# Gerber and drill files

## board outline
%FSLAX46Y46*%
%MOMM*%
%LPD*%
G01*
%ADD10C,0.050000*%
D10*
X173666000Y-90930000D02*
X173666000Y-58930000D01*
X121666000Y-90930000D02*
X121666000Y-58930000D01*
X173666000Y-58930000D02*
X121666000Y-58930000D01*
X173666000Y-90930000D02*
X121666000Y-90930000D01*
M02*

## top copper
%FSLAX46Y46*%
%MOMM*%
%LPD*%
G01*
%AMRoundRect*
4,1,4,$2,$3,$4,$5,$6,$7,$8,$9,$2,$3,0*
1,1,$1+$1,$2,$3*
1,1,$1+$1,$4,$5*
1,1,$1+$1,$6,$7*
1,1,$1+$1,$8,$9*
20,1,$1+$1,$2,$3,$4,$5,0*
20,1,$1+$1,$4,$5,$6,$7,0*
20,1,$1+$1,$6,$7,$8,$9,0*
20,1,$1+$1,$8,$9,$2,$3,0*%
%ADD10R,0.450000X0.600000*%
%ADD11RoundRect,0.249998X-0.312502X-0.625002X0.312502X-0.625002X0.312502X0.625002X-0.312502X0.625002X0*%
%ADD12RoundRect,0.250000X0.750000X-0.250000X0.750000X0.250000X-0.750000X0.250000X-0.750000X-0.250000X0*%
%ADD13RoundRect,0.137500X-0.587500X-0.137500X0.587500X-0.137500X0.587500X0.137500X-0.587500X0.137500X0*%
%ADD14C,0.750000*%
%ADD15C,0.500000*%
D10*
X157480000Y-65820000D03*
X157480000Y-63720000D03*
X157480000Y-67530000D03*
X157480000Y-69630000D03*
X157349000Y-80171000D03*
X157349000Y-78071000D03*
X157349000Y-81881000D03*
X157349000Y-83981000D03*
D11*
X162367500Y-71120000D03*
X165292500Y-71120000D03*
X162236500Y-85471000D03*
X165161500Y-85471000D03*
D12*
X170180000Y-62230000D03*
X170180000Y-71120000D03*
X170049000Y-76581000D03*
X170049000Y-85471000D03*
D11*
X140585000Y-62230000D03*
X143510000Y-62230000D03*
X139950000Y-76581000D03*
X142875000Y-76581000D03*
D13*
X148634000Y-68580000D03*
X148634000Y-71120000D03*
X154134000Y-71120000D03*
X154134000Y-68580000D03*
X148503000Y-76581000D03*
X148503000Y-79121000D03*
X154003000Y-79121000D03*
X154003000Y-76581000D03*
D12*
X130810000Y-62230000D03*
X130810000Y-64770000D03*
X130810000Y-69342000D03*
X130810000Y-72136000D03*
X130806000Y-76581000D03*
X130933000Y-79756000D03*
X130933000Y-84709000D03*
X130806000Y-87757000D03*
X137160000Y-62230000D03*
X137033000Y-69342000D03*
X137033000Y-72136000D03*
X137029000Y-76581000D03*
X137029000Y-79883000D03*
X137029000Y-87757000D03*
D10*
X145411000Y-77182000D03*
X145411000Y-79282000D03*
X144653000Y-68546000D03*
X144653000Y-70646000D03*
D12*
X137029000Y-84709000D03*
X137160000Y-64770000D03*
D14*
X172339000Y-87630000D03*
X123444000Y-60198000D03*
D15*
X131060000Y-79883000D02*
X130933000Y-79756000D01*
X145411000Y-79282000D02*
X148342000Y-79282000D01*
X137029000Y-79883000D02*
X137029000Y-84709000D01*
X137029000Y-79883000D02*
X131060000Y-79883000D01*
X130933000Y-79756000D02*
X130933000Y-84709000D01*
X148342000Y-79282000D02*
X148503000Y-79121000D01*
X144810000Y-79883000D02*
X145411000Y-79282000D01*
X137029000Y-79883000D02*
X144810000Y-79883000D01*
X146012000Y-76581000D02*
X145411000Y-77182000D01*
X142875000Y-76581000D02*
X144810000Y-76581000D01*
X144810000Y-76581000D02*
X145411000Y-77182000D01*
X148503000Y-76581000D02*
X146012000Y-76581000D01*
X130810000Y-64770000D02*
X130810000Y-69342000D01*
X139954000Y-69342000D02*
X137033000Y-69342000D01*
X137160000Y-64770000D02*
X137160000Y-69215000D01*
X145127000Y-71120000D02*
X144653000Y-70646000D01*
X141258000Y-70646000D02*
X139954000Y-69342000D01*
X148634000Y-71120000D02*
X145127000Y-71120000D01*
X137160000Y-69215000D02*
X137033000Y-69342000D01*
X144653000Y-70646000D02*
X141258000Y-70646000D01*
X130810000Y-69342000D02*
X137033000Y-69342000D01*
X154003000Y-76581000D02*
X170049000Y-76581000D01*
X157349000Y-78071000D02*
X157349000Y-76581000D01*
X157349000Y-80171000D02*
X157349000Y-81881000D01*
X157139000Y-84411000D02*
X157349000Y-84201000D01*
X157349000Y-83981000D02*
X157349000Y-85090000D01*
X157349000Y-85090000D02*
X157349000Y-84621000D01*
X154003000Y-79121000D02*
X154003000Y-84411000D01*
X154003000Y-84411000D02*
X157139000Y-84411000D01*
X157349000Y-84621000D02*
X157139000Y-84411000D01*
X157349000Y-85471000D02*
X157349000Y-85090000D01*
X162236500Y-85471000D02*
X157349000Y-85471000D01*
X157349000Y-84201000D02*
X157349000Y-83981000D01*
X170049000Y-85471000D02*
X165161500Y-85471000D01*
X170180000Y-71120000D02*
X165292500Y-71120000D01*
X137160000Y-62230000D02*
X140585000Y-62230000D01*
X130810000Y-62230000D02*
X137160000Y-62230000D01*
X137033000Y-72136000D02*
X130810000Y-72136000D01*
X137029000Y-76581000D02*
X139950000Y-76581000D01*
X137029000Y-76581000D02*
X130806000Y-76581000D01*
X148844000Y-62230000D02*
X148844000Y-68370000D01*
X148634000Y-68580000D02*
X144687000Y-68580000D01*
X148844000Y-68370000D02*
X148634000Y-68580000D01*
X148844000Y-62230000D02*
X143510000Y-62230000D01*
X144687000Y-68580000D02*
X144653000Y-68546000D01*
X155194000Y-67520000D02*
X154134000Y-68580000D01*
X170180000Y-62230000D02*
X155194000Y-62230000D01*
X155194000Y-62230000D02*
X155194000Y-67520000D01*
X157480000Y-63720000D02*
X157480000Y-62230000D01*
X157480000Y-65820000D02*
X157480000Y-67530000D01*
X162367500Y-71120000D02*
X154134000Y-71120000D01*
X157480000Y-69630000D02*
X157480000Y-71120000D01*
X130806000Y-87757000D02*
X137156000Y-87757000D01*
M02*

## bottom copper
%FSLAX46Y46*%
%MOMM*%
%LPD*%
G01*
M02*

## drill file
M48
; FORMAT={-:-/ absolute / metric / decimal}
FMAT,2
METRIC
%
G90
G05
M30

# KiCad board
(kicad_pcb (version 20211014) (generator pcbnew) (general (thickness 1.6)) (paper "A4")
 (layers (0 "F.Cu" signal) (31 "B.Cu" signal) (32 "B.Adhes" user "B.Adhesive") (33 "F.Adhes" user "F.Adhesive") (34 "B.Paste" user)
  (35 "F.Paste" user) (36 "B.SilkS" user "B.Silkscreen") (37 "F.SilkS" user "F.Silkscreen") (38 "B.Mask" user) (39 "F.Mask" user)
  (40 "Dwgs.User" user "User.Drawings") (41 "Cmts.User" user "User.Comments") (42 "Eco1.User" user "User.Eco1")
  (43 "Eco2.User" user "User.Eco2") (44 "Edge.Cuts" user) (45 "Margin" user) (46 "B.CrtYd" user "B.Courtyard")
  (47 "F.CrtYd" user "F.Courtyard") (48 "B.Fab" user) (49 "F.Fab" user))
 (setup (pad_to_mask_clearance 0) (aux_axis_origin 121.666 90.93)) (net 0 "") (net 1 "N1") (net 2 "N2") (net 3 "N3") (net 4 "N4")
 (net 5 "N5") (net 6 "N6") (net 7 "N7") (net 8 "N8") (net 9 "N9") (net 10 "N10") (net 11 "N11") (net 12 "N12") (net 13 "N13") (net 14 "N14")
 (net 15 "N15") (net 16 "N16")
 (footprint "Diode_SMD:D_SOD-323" (layer "F.Cu") (at 157.48 64.77 90)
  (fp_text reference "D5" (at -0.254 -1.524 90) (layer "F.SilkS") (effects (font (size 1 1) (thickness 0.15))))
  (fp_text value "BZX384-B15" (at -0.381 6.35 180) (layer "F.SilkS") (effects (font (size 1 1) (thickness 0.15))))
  (pad "1" smd rect locked (at -1.05 0 90) (size 0.6 0.45) (layers "F.Cu" "F.Paste" "F.Mask") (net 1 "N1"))
  (pad "2" smd rect locked (at 1.05 0 90) (size 0.6 0.45) (layers "F.Cu" "F.Paste" "F.Mask") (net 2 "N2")))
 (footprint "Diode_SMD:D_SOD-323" (layer "F.Cu") (at 157.48 68.58 -90)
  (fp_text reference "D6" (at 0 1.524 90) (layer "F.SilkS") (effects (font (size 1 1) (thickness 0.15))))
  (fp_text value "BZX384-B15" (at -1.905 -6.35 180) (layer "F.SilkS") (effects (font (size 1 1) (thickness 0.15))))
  (pad "1" smd rect locked (at -1.05 0 270) (size 0.6 0.45) (layers "F.Cu" "F.Paste" "F.Mask") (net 1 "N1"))
  (pad "2" smd rect locked (at 1.05 0 270) (size 0.6 0.45) (layers "F.Cu" "F.Paste" "F.Mask") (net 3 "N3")))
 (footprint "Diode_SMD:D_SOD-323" (layer "F.Cu") (at 157.349 79.121 90)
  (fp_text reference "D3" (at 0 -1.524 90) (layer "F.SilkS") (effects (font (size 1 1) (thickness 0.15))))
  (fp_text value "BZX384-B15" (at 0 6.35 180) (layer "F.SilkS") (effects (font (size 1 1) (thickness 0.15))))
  (pad "1" smd rect locked (at -1.05 0 90) (size 0.6 0.45) (layers "F.Cu" "F.Paste" "F.Mask") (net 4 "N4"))
  (pad "2" smd rect locked (at 1.05 0 90) (size 0.6 0.45) (layers "F.Cu" "F.Paste" "F.Mask") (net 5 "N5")))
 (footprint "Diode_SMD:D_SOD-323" (layer "F.Cu") (at 157.349 82.931 -90)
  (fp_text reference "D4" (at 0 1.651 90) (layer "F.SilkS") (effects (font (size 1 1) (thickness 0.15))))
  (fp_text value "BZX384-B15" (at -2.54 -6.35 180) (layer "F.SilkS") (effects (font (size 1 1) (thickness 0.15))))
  (pad "1" smd rect locked (at -1.05 0 270) (size 0.6 0.45) (layers "F.Cu" "F.Paste" "F.Mask") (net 4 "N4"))
  (pad "2" smd rect locked (at 1.05 0 270) (size 0.6 0.45) (layers "F.Cu" "F.Paste" "F.Mask") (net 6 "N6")))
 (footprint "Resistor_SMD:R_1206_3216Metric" (layer "F.Cu") (at 163.83 71.12)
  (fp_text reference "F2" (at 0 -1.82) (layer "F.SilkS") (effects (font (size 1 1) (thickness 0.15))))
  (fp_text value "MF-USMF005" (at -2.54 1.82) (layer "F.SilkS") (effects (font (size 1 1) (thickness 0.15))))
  (pad "1" smd roundrect locked (at -1.4625 0) (size 1.125 1.75) (layers "F.Cu" "F.Paste" "F.Mask") (roundrect_rratio 0.2222204444)
   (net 3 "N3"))
  (pad "2" smd roundrect locked (at 1.4625 0) (size 1.125 1.75) (layers "F.Cu" "F.Paste" "F.Mask") (roundrect_rratio 0.2222204444)
   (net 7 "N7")))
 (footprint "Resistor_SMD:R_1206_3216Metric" (layer "F.Cu") (at 163.699 85.471)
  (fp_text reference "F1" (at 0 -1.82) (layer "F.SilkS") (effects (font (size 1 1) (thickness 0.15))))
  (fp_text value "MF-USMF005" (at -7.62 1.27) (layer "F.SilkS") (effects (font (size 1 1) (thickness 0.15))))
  (pad "1" smd roundrect locked (at -1.4625 0) (size 1.125 1.75) (layers "F.Cu" "F.Paste" "F.Mask") (roundrect_rratio 0.2222204444)
   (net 6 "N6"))
  (pad "2" smd roundrect locked (at 1.4625 0) (size 1.125 1.75) (layers "F.Cu" "F.Paste" "F.Mask") (roundrect_rratio 0.2222204444)
   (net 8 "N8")))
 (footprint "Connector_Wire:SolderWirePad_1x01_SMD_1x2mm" (layer "F.Cu") (at 170.18 62.23 90)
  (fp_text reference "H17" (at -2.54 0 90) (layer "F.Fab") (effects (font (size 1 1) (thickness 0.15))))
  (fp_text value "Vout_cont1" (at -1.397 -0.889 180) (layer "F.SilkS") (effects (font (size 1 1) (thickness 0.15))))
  (pad "1" smd roundrect locked (at 0 0 90) (size 1 2) (layers "F.Cu" "F.Paste" "F.Mask") (roundrect_rratio 0.25) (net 2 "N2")))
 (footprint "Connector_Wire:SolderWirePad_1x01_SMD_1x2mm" (layer "F.Cu") (at 170.18 71.12 90)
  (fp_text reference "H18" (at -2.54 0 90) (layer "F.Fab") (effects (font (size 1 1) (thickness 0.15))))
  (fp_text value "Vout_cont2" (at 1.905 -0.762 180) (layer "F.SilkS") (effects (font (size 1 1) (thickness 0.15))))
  (pad "1" smd roundrect locked (at 0 0 90) (size 1 2) (layers "F.Cu" "F.Paste" "F.Mask") (roundrect_rratio 0.25) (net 7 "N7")))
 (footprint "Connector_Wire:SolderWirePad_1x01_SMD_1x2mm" (layer "F.Cu") (at 170.049 76.581 90)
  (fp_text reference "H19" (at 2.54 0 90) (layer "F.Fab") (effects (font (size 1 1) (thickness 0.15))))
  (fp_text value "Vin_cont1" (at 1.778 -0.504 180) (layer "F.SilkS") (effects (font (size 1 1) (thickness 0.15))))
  (pad "1" smd roundrect locked (at 0 0 90) (size 1 2) (layers "F.Cu" "F.Paste" "F.Mask") (roundrect_rratio 0.25) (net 5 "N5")))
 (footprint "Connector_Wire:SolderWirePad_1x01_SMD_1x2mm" (layer "F.Cu") (at 170.049 85.471 90)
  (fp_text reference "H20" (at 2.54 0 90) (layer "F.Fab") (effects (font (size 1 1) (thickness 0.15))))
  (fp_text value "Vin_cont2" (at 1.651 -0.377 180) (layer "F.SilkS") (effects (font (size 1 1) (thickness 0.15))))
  (pad "1" smd roundrect locked (at 0 0 90) (size 1 2) (layers "F.Cu" "F.Paste" "F.Mask") (roundrect_rratio 0.25) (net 8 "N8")))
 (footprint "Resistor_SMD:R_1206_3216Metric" (layer "F.Cu") (at 142.0475 62.23)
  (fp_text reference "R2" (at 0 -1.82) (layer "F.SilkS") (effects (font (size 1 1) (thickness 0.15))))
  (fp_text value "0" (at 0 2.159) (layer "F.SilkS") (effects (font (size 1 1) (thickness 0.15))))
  (pad "1" smd roundrect locked (at -1.4625 0) (size 1.125 1.75) (layers "F.Cu" "F.Paste" "F.Mask") (roundrect_rratio 0.2222204444)
   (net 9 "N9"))
  (pad "2" smd roundrect locked (at 1.4625 0) (size 1.125 1.75) (layers "F.Cu" "F.Paste" "F.Mask") (roundrect_rratio 0.2222204444)
   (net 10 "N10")))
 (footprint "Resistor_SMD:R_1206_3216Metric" (layer "F.Cu") (at 141.4125 76.581)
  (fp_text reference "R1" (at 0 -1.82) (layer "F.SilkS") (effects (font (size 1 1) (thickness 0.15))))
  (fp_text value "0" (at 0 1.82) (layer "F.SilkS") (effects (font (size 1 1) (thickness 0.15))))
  (pad "1" smd roundrect locked (at -1.4625 0) (size 1.125 1.75) (layers "F.Cu" "F.Paste" "F.Mask") (roundrect_rratio 0.2222204444)
   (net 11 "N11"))
  (pad "2" smd roundrect locked (at 1.4625 0) (size 1.125 1.75) (layers "F.Cu" "F.Paste" "F.Mask") (roundrect_rratio 0.2222204444)
   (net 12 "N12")))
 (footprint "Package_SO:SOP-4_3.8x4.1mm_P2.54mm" (layer "F.Cu") (at 151.384 69.85)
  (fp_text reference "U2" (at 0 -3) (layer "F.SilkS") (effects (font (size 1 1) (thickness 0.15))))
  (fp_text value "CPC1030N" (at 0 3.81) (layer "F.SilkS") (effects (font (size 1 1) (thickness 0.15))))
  (pad "1" smd roundrect locked (at -2.75 -1.27) (size 1.45 0.55) (layers "F.Cu" "F.Paste" "F.Mask") (roundrect_rratio 0.25) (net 10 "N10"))
  (pad "2" smd roundrect locked (at -2.75 1.27) (size 1.45 0.55) (layers "F.Cu" "F.Paste" "F.Mask") (roundrect_rratio 0.25) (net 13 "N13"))
  (pad "3" smd roundrect locked (at 2.75 1.27) (size 1.45 0.55) (layers "F.Cu" "F.Paste" "F.Mask") (roundrect_rratio 0.25) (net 3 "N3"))
  (pad "4" smd roundrect locked (at 2.75 -1.27) (size 1.45 0.55) (layers "F.Cu" "F.Paste" "F.Mask") (roundrect_rratio 0.25) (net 2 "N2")))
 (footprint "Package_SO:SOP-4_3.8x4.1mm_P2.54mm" (layer "F.Cu") (at 151.253 77.851)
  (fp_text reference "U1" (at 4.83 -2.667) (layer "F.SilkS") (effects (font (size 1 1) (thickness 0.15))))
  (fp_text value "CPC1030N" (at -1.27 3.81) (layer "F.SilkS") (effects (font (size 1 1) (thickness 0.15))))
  (pad "1" smd roundrect locked (at -2.75 -1.27) (size 1.45 0.55) (layers "F.Cu" "F.Paste" "F.Mask") (roundrect_rratio 0.25) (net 12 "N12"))
  (pad "2" smd roundrect locked (at -2.75 1.27) (size 1.45 0.55) (layers "F.Cu" "F.Paste" "F.Mask") (roundrect_rratio 0.25) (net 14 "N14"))
  (pad "3" smd roundrect locked (at 2.75 1.27) (size 1.45 0.55) (layers "F.Cu" "F.Paste" "F.Mask") (roundrect_rratio 0.25) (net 6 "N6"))
  (pad "4" smd roundrect locked (at 2.75 -1.27) (size 1.45 0.55) (layers "F.Cu" "F.Paste" "F.Mask") (roundrect_rratio 0.25) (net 5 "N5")))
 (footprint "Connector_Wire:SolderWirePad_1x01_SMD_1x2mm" (layer "F.Cu") (at 130.81 62.23 90)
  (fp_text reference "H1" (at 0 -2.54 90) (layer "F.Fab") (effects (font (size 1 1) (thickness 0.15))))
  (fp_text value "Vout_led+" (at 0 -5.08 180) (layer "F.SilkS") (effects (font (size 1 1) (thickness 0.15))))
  (pad "1" smd roundrect locked (at 0 0 90) (size 1 2) (layers "F.Cu" "F.Paste" "F.Mask") (roundrect_rratio 0.25) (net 9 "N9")))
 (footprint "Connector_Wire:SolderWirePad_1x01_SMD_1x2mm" (layer "F.Cu") (at 130.81 64.77 90)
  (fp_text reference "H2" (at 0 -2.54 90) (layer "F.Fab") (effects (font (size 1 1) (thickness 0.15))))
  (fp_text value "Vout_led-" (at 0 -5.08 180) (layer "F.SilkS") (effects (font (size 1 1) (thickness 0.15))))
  (pad "1" smd roundrect locked (at 0 0 90) (size 1 2) (layers "F.Cu" "F.Paste" "F.Mask") (roundrect_rratio 0.25) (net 13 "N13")))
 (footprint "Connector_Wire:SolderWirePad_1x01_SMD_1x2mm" (layer "F.Cu") (at 130.81 69.342 90)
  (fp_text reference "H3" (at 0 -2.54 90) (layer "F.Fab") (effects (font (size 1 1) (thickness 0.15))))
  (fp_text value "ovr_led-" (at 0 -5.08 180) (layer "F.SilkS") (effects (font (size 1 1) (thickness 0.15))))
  (pad "1" smd roundrect locked (at 0 0 90) (size 1 2) (layers "F.Cu" "F.Paste" "F.Mask") (roundrect_rratio 0.25) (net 13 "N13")))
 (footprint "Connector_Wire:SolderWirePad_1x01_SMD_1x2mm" (layer "F.Cu") (at 130.81 72.136 90)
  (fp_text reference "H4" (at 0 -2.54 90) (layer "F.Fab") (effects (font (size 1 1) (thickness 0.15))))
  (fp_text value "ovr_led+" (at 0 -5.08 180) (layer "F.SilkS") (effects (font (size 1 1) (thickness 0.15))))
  (pad "1" smd roundrect locked (at 0 0 90) (size 1 2) (layers "F.Cu" "F.Paste" "F.Mask") (roundrect_rratio 0.25) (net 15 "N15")))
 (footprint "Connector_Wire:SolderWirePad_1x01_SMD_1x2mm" (layer "F.Cu") (at 130.806 76.581 90)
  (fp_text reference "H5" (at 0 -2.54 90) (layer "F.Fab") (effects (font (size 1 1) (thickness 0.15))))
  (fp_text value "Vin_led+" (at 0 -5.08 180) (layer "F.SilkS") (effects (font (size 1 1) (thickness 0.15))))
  (pad "1" smd roundrect locked (at 0 0 90) (size 1 2) (layers "F.Cu" "F.Paste" "F.Mask") (roundrect_rratio 0.25) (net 11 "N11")))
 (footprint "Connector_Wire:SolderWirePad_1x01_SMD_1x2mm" (layer "F.Cu") (at 130.933 79.756 90)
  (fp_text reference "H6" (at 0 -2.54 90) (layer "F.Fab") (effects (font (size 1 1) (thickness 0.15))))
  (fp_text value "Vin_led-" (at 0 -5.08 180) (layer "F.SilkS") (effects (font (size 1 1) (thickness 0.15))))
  (pad "1" smd roundrect locked (at 0 0 90) (size 1 2) (layers "F.Cu" "F.Paste" "F.Mask") (roundrect_rratio 0.25) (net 14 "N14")))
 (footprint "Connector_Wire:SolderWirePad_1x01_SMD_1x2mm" (layer "F.Cu") (at 130.933 84.709 90)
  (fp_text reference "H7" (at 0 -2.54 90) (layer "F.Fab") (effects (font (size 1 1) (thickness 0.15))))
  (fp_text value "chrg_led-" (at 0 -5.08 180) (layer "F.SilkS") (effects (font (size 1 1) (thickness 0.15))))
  (pad "1" smd roundrect locked (at 0 0 90) (size 1 2) (layers "F.Cu" "F.Paste" "F.Mask") (roundrect_rratio 0.25) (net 14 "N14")))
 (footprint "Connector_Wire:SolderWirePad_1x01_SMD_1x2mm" (layer "F.Cu") (at 130.806 87.757 90)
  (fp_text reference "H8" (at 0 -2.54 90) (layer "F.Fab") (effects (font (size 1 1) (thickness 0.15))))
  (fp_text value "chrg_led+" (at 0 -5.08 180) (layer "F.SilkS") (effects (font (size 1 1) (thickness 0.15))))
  (pad "1" smd roundrect locked (at 0 0 90) (size 1 2) (layers "F.Cu" "F.Paste" "F.Mask") (roundrect_rratio 0.25) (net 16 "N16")))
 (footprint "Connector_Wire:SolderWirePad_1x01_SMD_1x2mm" (layer "F.Cu") (at 137.16 62.23 90)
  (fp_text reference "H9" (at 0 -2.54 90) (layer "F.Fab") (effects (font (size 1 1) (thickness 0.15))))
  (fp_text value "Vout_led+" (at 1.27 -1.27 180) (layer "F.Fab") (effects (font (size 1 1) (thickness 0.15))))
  (pad "1" smd roundrect locked (at 0 0 90) (size 1 2) (layers "F.Cu" "F.Paste" "F.Mask") (roundrect_rratio 0.25) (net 9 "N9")))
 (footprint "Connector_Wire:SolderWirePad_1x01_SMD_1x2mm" (layer "F.Cu") (at 137.033 69.342 90)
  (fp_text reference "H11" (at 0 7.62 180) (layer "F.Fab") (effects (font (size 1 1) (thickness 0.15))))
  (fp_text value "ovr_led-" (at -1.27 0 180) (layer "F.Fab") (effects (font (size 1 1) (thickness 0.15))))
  (pad "1" smd roundrect locked (at 0 0 90) (size 1 2) (layers "F.Cu" "F.Paste" "F.Mask") (roundrect_rratio 0.25) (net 13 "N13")))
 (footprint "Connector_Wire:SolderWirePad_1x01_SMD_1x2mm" (layer "F.Cu") (at 137.033 72.136 90)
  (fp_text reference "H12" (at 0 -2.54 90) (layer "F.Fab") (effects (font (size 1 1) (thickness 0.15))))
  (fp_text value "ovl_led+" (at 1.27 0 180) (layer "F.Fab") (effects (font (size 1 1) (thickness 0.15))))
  (pad "1" smd roundrect locked (at 0 0 90) (size 1 2) (layers "F.Cu" "F.Paste" "F.Mask") (roundrect_rratio 0.25) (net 15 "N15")))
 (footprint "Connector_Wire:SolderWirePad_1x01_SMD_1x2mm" (layer "F.Cu") (at 137.029 76.581 90)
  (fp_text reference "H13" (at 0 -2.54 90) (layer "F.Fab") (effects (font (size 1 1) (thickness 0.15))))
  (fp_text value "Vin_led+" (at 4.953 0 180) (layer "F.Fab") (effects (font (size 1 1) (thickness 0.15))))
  (pad "1" smd roundrect locked (at 0 0 90) (size 1 2) (layers "F.Cu" "F.Paste" "F.Mask") (roundrect_rratio 0.25) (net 11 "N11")))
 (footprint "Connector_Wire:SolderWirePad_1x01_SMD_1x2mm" (layer "F.Cu") (at 137.029 79.883 90)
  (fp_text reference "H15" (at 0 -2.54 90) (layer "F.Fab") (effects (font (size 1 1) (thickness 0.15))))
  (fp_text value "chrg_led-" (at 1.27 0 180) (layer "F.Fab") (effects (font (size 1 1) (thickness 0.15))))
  (pad "1" smd roundrect locked (at 0 0 90) (size 1 2) (layers "F.Cu" "F.Paste" "F.Mask") (roundrect_rratio 0.25) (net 14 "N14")))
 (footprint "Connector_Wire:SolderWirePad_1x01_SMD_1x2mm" (layer "F.Cu") (at 137.029 87.757 90)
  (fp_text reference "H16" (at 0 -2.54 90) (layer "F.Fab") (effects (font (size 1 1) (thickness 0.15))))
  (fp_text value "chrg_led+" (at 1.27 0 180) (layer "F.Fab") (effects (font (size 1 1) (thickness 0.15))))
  (pad "1" smd roundrect locked (at 0 0 90) (size 1 2) (layers "F.Cu" "F.Paste" "F.Mask") (roundrect_rratio 0.25) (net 16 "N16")))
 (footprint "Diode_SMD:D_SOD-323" (layer "F.Cu") (at 145.411 78.232 -90)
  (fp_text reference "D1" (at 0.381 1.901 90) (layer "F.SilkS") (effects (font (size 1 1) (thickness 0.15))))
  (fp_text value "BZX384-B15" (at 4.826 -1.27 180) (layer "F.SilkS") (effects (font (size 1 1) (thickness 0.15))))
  (pad "1" smd rect locked (at -1.05 0 270) (size 0.6 0.45) (layers "F.Cu" "F.Paste" "F.Mask") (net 12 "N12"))
  (pad "2" smd rect locked (at 1.05 0 270) (size 0.6 0.45) (layers "F.Cu" "F.Paste" "F.Mask") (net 14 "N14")))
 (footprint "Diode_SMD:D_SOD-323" (layer "F.Cu") (at 144.653 69.596 -90)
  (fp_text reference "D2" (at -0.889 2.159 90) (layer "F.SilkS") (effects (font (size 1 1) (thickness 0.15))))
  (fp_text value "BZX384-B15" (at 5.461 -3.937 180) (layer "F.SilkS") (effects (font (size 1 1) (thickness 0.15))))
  (pad "1" smd rect locked (at -1.05 0 270) (size 0.6 0.45) (layers "F.Cu" "F.Paste" "F.Mask") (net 10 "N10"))
  (pad "2" smd rect locked (at 1.05 0 270) (size 0.6 0.45) (layers "F.Cu" "F.Paste" "F.Mask") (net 13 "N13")))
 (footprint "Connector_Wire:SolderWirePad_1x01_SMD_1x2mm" (layer "F.Cu") (at 137.029 84.709 90)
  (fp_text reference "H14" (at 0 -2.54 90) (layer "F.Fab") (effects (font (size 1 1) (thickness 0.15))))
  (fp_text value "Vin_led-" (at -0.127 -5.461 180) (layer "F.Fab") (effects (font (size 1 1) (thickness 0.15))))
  (pad "1" smd roundrect locked (at 0 0 90) (size 1 2) (layers "F.Cu" "F.Paste" "F.Mask") (roundrect_rratio 0.25) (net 14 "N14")))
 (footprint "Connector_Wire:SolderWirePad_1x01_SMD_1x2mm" (layer "F.Cu") (at 137.16 64.77 90)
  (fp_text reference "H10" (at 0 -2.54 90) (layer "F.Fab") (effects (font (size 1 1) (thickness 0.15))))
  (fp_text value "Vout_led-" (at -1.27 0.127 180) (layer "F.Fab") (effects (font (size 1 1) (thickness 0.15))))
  (pad "1" smd roundrect locked (at 0 0 90) (size 1 2) (layers "F.Cu" "F.Paste" "F.Mask") (roundrect_rratio 0.25) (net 13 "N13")))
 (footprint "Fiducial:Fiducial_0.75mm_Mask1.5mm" (layer "F.Cu") (at 172.339 87.63)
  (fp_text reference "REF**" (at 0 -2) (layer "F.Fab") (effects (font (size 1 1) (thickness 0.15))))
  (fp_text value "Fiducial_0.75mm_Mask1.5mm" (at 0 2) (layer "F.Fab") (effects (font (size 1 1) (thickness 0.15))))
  (pad "" smd circle locked (at 0 0) (size 0.75 0.75) (layers "F.Cu" "F.Mask") (solder_mask_margin 0.375) (clearance 0.375)))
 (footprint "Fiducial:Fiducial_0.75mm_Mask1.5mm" (layer "F.Cu") (at 123.444 60.198)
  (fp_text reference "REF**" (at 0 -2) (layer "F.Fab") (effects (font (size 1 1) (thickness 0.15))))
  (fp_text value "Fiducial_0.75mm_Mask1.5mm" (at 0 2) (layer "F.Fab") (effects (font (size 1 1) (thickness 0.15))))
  (pad "" smd circle locked (at 0 0) (size 0.75 0.75) (layers "F.Cu" "F.Mask") (solder_mask_margin 0.375) (clearance 0.375)))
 (gr_line (start 173.666 90.93) (end 173.666 58.93) (layer "Edge.Cuts") (width 0.05))
 (gr_line (start 121.666 90.93) (end 121.666 58.93) (layer "Edge.Cuts") (width 0.05))
 (gr_line (start 173.666 58.93) (end 121.666 58.93) (layer "Edge.Cuts") (width 0.05))
 (gr_line (start 173.666 90.93) (end 121.666 90.93) (layer "Edge.Cuts") (width 0.05))
 (segment (start 131.06 79.883) (end 130.933 79.756) (width 0.5) (layer "F.Cu") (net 14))
 (segment (start 145.411 79.282) (end 148.342 79.282) (width 0.5) (layer "F.Cu") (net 14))
 (segment (start 137.029 79.883) (end 137.029 84.709) (width 0.5) (layer "F.Cu") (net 14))
 (segment (start 137.029 79.883) (end 131.06 79.883) (width 0.5) (layer "F.Cu") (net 14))
 (segment (start 130.933 79.756) (end 130.933 84.709) (width 0.5) (layer "F.Cu") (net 14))
 (segment (start 148.342 79.282) (end 148.503 79.121) (width 0.5) (layer "F.Cu") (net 14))
 (segment (start 144.81 79.883) (end 145.411 79.282) (width 0.5) (layer "F.Cu") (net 14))
 (segment (start 137.029 79.883) (end 144.81 79.883) (width 0.5) (layer "F.Cu") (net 14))
 (segment (start 146.012 76.581) (end 145.411 77.182) (width 0.5) (layer "F.Cu") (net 12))
 (segment (start 142.875 76.581) (end 144.81 76.581) (width 0.5) (layer "F.Cu") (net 12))
 (segment (start 144.81 76.581) (end 145.411 77.182) (width 0.5) (layer "F.Cu") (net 12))
 (segment (start 148.503 76.581) (end 146.012 76.581) (width 0.5) (layer "F.Cu") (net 12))
 (segment (start 130.81 64.77) (end 130.81 69.342) (width 0.5) (layer "F.Cu") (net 13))
 (segment (start 139.954 69.342) (end 137.033 69.342) (width 0.5) (layer "F.Cu") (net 13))
 (segment (start 137.16 64.77) (end 137.16 69.215) (width 0.5) (layer "F.Cu") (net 13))
 (segment (start 145.127 71.12) (end 144.653 70.646) (width 0.5) (layer "F.Cu") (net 13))
 (segment (start 141.258 70.646) (end 139.954 69.342) (width 0.5) (layer "F.Cu") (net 13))
 (segment (start 148.634 71.12) (end 145.127 71.12) (width 0.5) (layer "F.Cu") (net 13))
 (segment (start 137.16 69.215) (end 137.033 69.342) (width 0.5) (layer "F.Cu") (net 13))
 (segment (start 144.653 70.646) (end 141.258 70.646) (width 0.5) (layer "F.Cu") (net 13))
 (segment (start 130.81 69.342) (end 137.033 69.342) (width 0.5) (layer "F.Cu") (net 13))
 (segment (start 154.003 76.581) (end 170.049 76.581) (width 0.5) (layer "F.Cu") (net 5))
 (segment (start 157.349 78.071) (end 157.349 76.581) (width 0.5) (layer "F.Cu") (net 5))
 (segment (start 157.349 80.171) (end 157.349 81.881) (width 0.5) (layer "F.Cu") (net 4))
 (segment (start 157.139 84.411) (end 157.349 84.201) (width 0.5) (layer "F.Cu") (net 6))
 (segment (start 157.349 83.981) (end 157.349 85.09) (width 0.5) (layer "F.Cu") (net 6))
 (segment (start 157.349 85.09) (end 157.349 84.621) (width 0.5) (layer "F.Cu") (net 6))
 (segment (start 154.003 79.121) (end 154.003 84.411) (width 0.5) (layer "F.Cu") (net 6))
 (segment (start 154.003 84.411) (end 157.139 84.411) (width 0.5) (layer "F.Cu") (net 6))
 (segment (start 157.349 84.621) (end 157.139 84.411) (width 0.5) (layer "F.Cu") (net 6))
 (segment (start 157.349 85.471) (end 157.349 85.09) (width 0.5) (layer "F.Cu") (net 6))
 (segment (start 162.2365 85.471) (end 157.349 85.471) (width 0.5) (layer "F.Cu") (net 6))
 (segment (start 157.349 84.201) (end 157.349 83.981) (width 0.5) (layer "F.Cu") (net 6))
 (segment (start 170.049 85.471) (end 165.1615 85.471) (width 0.5) (layer "F.Cu") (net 8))
 (segment (start 170.18 71.12) (end 165.2925 71.12) (width 0.5) (layer "F.Cu") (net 7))
 (segment (start 137.16 62.23) (end 140.585 62.23) (width 0.5) (layer "F.Cu") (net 9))
 (segment (start 130.81 62.23) (end 137.16 62.23) (width 0.5) (layer "F.Cu") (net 9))
 (segment (start 137.033 72.136) (end 130.81 72.136) (width 0.5) (layer "F.Cu") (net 15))
 (segment (start 137.029 76.581) (end 139.95 76.581) (width 0.5) (layer "F.Cu") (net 11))
 (segment (start 137.029 76.581) (end 130.806 76.581) (width 0.5) (layer "F.Cu") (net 11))
 (segment (start 148.844 62.23) (end 148.844 68.37) (width 0.5) (layer "F.Cu") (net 10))
 (segment (start 148.634 68.58) (end 144.687 68.58) (width 0.5) (layer "F.Cu") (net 10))
 (segment (start 148.844 68.37) (end 148.634 68.58) (width 0.5) (layer "F.Cu") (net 10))
 (segment (start 148.844 62.23) (end 143.51 62.23) (width 0.5) (layer "F.Cu") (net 10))
 (segment (start 144.687 68.58) (end 144.653 68.546) (width 0.5) (layer "F.Cu") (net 10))
 (segment (start 155.194 67.52) (end 154.134 68.58) (width 0.5) (layer "F.Cu") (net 2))
 (segment (start 170.18 62.23) (end 155.194 62.23) (width 0.5) (layer "F.Cu") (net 2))
 (segment (start 155.194 62.23) (end 155.194 67.52) (width 0.5) (layer "F.Cu") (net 2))
 (segment (start 157.48 63.72) (end 157.48 62.23) (width 0.5) (layer "F.Cu") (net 2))
 (segment (start 157.48 65.82) (end 157.48 67.53) (width 0.5) (layer "F.Cu") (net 1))
 (segment (start 162.3675 71.12) (end 154.134 71.12) (width 0.5) (layer "F.Cu") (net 3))
 (segment (start 157.48 69.63) (end 157.48 71.12) (width 0.5) (layer "F.Cu") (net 3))
 (segment (start 130.806 87.757) (end 137.156 87.757) (width 0.5) (layer "F.Cu") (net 16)))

